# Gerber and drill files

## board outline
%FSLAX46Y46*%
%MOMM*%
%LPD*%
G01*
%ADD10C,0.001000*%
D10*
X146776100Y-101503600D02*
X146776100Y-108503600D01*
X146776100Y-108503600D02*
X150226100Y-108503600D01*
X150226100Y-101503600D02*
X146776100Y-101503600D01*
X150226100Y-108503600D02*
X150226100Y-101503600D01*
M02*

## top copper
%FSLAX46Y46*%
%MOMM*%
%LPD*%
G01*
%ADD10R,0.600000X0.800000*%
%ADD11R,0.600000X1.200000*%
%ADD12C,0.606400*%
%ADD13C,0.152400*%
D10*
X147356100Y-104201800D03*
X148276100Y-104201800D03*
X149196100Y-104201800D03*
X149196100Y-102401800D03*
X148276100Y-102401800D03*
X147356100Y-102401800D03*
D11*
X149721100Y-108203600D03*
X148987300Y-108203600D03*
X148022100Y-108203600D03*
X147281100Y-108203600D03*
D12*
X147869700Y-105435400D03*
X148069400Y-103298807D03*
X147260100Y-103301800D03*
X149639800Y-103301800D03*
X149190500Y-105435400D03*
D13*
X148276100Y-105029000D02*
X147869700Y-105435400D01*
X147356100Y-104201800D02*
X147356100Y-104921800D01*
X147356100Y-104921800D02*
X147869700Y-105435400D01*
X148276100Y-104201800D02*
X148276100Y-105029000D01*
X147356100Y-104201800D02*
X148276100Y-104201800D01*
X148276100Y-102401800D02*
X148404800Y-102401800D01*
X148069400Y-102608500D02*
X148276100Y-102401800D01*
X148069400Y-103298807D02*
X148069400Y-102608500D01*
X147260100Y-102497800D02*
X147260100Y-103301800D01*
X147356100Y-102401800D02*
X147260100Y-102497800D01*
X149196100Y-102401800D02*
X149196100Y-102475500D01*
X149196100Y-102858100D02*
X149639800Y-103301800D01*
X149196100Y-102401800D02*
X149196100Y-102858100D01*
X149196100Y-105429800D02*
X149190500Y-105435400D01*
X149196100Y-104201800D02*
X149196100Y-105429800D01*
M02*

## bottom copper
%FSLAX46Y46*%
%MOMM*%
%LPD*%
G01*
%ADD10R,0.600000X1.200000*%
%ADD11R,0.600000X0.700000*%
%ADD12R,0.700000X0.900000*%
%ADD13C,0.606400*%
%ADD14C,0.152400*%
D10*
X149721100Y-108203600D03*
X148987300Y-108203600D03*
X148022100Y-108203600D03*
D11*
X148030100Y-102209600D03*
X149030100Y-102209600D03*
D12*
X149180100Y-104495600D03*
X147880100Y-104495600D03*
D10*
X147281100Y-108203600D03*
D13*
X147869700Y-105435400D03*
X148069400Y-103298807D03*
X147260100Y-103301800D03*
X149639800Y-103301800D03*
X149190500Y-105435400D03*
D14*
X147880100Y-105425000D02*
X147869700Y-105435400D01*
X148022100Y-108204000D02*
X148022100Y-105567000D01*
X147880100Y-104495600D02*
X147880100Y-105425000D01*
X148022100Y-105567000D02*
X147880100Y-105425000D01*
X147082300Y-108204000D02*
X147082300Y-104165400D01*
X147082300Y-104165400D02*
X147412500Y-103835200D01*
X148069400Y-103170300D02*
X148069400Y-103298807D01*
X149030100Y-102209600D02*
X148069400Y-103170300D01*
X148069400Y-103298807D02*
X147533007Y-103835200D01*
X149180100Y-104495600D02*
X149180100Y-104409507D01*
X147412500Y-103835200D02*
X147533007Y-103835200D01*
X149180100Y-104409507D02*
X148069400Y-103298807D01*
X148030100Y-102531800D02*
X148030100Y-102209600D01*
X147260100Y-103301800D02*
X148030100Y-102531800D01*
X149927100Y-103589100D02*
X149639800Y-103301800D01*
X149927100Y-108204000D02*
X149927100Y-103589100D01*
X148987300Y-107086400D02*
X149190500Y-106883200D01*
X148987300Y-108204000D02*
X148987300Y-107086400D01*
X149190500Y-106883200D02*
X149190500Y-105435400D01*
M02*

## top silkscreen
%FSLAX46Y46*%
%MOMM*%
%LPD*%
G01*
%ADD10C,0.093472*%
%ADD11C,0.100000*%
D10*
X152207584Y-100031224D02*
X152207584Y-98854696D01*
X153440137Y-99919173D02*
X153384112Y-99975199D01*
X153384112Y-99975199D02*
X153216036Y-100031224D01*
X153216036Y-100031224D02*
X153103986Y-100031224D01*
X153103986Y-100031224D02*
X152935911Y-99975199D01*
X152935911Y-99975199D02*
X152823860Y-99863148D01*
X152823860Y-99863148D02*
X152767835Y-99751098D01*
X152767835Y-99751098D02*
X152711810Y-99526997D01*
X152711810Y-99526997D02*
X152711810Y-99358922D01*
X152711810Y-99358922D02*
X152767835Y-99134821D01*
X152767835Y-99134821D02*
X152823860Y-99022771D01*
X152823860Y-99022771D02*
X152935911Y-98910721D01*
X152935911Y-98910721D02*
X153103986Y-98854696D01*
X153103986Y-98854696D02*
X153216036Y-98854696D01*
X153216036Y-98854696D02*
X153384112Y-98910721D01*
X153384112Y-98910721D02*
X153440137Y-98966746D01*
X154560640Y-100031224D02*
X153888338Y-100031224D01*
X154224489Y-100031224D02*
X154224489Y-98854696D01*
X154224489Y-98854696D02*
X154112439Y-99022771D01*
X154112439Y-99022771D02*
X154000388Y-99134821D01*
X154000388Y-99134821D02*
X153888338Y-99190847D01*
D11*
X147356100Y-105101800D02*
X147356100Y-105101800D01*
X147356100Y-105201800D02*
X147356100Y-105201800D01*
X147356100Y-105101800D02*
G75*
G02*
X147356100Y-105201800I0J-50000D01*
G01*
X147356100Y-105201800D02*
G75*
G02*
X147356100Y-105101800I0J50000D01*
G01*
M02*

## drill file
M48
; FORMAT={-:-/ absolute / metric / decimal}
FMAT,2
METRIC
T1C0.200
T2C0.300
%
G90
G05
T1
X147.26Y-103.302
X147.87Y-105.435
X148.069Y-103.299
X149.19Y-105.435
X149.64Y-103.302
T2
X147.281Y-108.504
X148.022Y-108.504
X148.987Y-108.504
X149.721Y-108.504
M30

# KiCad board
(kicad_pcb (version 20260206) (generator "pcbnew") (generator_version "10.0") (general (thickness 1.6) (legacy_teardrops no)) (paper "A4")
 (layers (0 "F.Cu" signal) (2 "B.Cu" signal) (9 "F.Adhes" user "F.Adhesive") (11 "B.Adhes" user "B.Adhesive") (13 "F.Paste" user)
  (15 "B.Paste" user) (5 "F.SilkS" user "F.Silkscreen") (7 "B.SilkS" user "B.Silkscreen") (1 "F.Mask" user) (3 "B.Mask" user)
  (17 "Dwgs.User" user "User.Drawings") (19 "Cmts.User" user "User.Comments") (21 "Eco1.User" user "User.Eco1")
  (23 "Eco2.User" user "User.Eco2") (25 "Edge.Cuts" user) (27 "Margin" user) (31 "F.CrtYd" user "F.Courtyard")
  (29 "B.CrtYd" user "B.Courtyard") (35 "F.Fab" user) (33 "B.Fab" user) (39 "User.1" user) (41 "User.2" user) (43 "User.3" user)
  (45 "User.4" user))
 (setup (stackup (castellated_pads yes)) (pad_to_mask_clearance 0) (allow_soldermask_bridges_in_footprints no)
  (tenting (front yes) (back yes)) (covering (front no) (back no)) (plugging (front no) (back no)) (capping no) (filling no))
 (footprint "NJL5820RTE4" (layer "F.Cu") (at 148.2761 103.3018)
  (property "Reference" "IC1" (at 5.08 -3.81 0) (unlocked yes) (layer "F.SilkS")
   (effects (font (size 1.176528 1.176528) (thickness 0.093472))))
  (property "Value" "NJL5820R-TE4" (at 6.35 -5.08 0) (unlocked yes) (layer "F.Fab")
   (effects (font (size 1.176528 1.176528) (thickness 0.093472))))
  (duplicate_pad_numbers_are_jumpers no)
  (fp_line (start -0.92 1.8) (end -0.92 1.8) (stroke (width 0.1) (type solid)) (layer "F.SilkS"))
  (fp_line (start -0.92 1.9) (end -0.92 1.9) (stroke (width 0.1) (type solid)) (layer "F.SilkS"))
  (fp_arc (start -0.92 1.8) (mid -0.87 1.85) (end -0.92 1.9) (stroke (width 0.1) (type solid)) (layer "F.SilkS"))
  (fp_arc (start -0.92 1.9) (mid -0.97 1.85) (end -0.92 1.8) (stroke (width 0.1) (type solid)) (layer "F.SilkS"))
  (pad "1" smd rect (at -0.92 0.9 90) (size 0.8 0.6) (layers "F.Cu" "F.Mask" "F.Paste") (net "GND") (solder_mask_margin 0.1016)
   (solder_paste_margin 0) (thermal_bridge_angle 0))
  (pad "2" smd rect (at 0 0.9 90) (size 0.8 0.6) (layers "F.Cu" "F.Mask" "F.Paste") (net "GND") (solder_mask_margin 0.1016)
   (solder_paste_margin 0) (thermal_bridge_angle 0))
  (pad "3" smd rect (at 0.92 0.9 90) (size 0.8 0.6) (layers "F.Cu" "F.Mask" "F.Paste") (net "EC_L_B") (solder_mask_margin 0.1016)
   (solder_paste_margin 0) (thermal_bridge_angle 0))
  (pad "4" smd rect (at 0.92 -0.9 90) (size 0.8 0.6) (layers "F.Cu" "F.Mask" "F.Paste") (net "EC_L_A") (solder_mask_margin 0.1016)
   (solder_paste_margin 0) (thermal_bridge_angle 0))
  (pad "5" smd rect (at 0 -0.9 90) (size 0.8 0.6) (layers "F.Cu" "F.Mask" "F.Paste") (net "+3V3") (solder_mask_margin 0.1016)
   (solder_paste_margin 0) (thermal_bridge_angle 0))
  (pad "6" smd rect (at -0.92 -0.9 90) (size 0.8 0.6) (layers "F.Cu" "F.Mask" "F.Paste") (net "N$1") (solder_mask_margin 0.1016)
   (solder_paste_margin 0) (thermal_bridge_angle 0)))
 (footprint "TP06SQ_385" (layer "B.Cu") (at 149.9271 108.204 180)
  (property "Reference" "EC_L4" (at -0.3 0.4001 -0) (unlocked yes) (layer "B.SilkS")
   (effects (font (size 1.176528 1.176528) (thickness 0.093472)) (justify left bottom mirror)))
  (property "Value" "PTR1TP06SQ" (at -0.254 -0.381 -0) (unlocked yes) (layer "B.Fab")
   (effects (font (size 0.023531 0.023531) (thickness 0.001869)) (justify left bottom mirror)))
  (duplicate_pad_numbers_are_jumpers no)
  (pad "TP" thru_hole rect (at 0.2060 -0.2996 180) (size 0.6 1.2) (drill 0.3 (offset 0 0.3000)) (layers "*.Cu" "*.Mask") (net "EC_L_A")
   (solder_mask_margin 0) (solder_paste_margin 0) (thermal_bridge_angle 0)))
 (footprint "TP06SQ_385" (layer "B.Cu") (at 148.9873 108.204 180)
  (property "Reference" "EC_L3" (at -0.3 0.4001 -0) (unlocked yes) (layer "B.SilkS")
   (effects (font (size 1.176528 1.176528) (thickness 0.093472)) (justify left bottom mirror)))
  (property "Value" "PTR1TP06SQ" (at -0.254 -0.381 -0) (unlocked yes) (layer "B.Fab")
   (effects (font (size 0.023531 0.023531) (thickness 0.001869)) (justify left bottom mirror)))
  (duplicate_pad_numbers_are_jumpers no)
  (pad "TP" thru_hole rect (at 0 -0.2996 180) (size 0.6 1.2) (drill 0.3 (offset 0 0.3000)) (layers "*.Cu" "*.Mask") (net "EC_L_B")
   (solder_mask_margin 0) (solder_paste_margin 0) (thermal_bridge_angle 0)))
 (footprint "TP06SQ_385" (layer "B.Cu") (at 148.0221 108.204 180)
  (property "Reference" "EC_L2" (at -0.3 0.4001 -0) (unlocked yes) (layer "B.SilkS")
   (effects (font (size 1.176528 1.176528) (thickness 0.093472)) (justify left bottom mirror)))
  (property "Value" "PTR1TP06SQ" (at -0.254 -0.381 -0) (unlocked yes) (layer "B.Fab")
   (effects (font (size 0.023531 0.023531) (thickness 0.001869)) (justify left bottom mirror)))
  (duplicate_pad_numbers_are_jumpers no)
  (pad "TP" thru_hole rect (at 0 -0.2996 180) (size 0.6 1.2) (drill 0.3 (offset 0 0.3000)) (layers "*.Cu" "*.Mask") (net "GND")
   (solder_mask_margin 0) (solder_paste_margin 0) (thermal_bridge_angle 0)))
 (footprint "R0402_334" (layer "B.Cu") (at 148.5301 102.2096)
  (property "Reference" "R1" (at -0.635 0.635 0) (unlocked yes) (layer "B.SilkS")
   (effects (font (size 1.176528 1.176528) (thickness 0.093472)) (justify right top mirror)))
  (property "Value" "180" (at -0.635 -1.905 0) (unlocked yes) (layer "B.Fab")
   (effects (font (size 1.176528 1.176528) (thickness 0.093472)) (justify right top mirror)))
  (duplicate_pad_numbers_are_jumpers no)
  (pad "1" smd rect (at -0.5 0) (size 0.6 0.7) (layers "B.Cu" "B.Mask" "B.Paste") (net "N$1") (solder_mask_margin 0.1016)
   (solder_paste_margin 0) (thermal_bridge_angle 0))
  (pad "2" smd rect (at 0.5 0) (size 0.6 0.7) (layers "B.Cu" "B.Mask" "B.Paste") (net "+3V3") (solder_mask_margin 0.1016)
   (solder_paste_margin 0) (thermal_bridge_angle 0)))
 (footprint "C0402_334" (layer "B.Cu") (at 148.5301 104.4956 180)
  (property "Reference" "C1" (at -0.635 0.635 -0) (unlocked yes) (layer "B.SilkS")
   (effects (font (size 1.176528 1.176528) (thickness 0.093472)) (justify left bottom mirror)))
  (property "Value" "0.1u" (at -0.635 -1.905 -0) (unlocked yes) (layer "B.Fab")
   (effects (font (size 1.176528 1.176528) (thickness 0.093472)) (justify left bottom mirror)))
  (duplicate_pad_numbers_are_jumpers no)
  (pad "1" smd rect (at -0.65 0 180) (size 0.7 0.9) (layers "B.Cu" "B.Mask" "B.Paste") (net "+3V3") (solder_mask_margin 0.1016)
   (solder_paste_margin 0) (thermal_bridge_angle 0))
  (pad "2" smd rect (at 0.65 0 180) (size 0.7 0.9) (layers "B.Cu" "B.Mask" "B.Paste") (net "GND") (solder_mask_margin 0.1016)
   (solder_paste_margin 0) (thermal_bridge_angle 0)))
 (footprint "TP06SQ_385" (layer "B.Cu") (at 147.0823 108.204 180)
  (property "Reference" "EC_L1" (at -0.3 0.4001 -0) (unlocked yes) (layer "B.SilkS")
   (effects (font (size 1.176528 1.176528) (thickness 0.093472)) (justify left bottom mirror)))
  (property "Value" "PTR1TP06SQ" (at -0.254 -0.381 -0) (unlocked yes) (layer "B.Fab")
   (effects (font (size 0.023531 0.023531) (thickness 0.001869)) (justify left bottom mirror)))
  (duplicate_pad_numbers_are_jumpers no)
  (pad "TP" thru_hole rect (at -0.1988 -0.2996 180) (size 0.6 1.2) (drill 0.3 (offset 0 0.3000)) (layers "*.Cu" "*.Mask") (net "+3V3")
   (solder_mask_margin 0) (solder_paste_margin 0) (thermal_bridge_angle 0)))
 (gr_line (start 146.7761 101.5036) (end 146.7761 108.5036) (stroke (width 0.001) (type solid)) (layer "Edge.Cuts"))
 (gr_line (start 146.7761 108.5036) (end 150.2261 108.5036) (stroke (width 0.001) (type solid)) (layer "Edge.Cuts"))
 (gr_line (start 150.2261 101.5036) (end 146.7761 101.5036) (stroke (width 0.001) (type solid)) (layer "Edge.Cuts"))
 (gr_line (start 150.2261 108.5036) (end 150.2261 101.5036) (stroke (width 0.001) (type solid)) (layer "Edge.Cuts"))
 (segment (start 148.2761 105.029) (end 147.8697 105.4354) (width 0.1524) (layer "F.Cu") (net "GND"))
 (segment (start 147.3561 104.2018) (end 147.3561 104.9218) (width 0.1524) (layer "F.Cu") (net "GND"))
 (segment (start 147.3561 104.9218) (end 147.8697 105.4354) (width 0.1524) (layer "F.Cu") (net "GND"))
 (segment (start 148.2761 104.2018) (end 148.2761 105.029) (width 0.1524) (layer "F.Cu") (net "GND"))
 (segment (start 147.3561 104.2018) (end 148.2761 104.2018) (width 0.1524) (layer "F.Cu") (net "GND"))
 (via (at 147.8697 105.4354) (size 0.6064) (drill 0.2) (layers "F.Cu" "B.Cu") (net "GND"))
 (segment (start 147.8801 105.425) (end 147.8697 105.4354) (width 0.1524) (layer "B.Cu") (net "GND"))
 (segment (start 148.0221 108.204) (end 148.0221 105.567) (width 0.1524) (layer "B.Cu") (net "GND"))
 (segment (start 147.8801 104.4956) (end 147.8801 105.425) (width 0.1524) (layer "B.Cu") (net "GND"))
 (segment (start 148.0221 105.567) (end 147.8801 105.425) (width 0.1524) (layer "B.Cu") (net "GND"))
 (segment (start 148.2761 102.4018) (end 148.4048 102.4018) (width 0.1524) (layer "F.Cu") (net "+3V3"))
 (segment (start 148.0694 102.6085) (end 148.2761 102.4018) (width 0.1524) (layer "F.Cu") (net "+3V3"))
 (segment (start 148.0694 103.298807) (end 148.0694 102.6085) (width 0.1524) (layer "F.Cu") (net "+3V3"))
 (via (at 148.0694 103.298807) (size 0.6064) (drill 0.2) (layers "F.Cu" "B.Cu") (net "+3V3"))
 (segment (start 147.0823 108.204) (end 147.0823 104.1654) (width 0.1524) (layer "B.Cu") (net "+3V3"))
 (segment (start 147.0823 104.1654) (end 147.4125 103.8352) (width 0.1524) (layer "B.Cu") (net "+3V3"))
 (segment (start 148.0694 103.1703) (end 148.0694 103.298807) (width 0.1524) (layer "B.Cu") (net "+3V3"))
 (segment (start 149.0301 102.2096) (end 148.0694 103.1703) (width 0.1524) (layer "B.Cu") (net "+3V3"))
 (segment (start 148.0694 103.298807) (end 147.533007 103.8352) (width 0.1524) (layer "B.Cu") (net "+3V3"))
 (segment (start 149.1801 104.4956) (end 149.1801 104.409507) (width 0.1524) (layer "B.Cu") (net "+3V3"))
 (segment (start 147.4125 103.8352) (end 147.533007 103.8352) (width 0.1524) (layer "B.Cu") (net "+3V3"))
 (segment (start 149.1801 104.409507) (end 148.0694 103.298807) (width 0.1524) (layer "B.Cu") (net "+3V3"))
 (segment (start 147.2601 102.4978) (end 147.2601 103.3018) (width 0.1524) (layer "F.Cu") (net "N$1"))
 (segment (start 147.3561 102.4018) (end 147.2601 102.4978) (width 0.1524) (layer "F.Cu") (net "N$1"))
 (via (at 147.2601 103.3018) (size 0.6064) (drill 0.2) (layers "F.Cu" "B.Cu") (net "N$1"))
 (segment (start 148.0301 102.5318) (end 148.0301 102.2096) (width 0.1524) (layer "B.Cu") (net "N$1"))
 (segment (start 147.2601 103.3018) (end 148.0301 102.5318) (width 0.1524) (layer "B.Cu") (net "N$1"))
 (segment (start 149.1961 102.4018) (end 149.1961 102.4755) (width 0.1524) (layer "F.Cu") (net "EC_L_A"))
 (segment (start 149.1961 102.8581) (end 149.6398 103.3018) (width 0.1524) (layer "F.Cu") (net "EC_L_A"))
 (segment (start 149.1961 102.4018) (end 149.1961 102.8581) (width 0.1524) (layer "F.Cu") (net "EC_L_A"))
 (via (at 149.6398 103.3018) (size 0.6064) (drill 0.2) (layers "F.Cu" "B.Cu") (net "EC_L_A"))
 (segment (start 149.9271 103.5891) (end 149.6398 103.3018) (width 0.1524) (layer "B.Cu") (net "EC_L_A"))
 (segment (start 149.9271 108.204) (end 149.9271 103.5891) (width 0.1524) (layer "B.Cu") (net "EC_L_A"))
 (segment (start 149.1961 105.4298) (end 149.1905 105.4354) (width 0.1524) (layer "F.Cu") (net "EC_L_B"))
 (segment (start 149.1961 104.2018) (end 149.1961 105.4298) (width 0.1524) (layer "F.Cu") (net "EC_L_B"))
 (via (at 149.1905 105.4354) (size 0.6064) (drill 0.2) (layers "F.Cu" "B.Cu") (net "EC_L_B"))
 (segment (start 148.9873 107.0864) (end 149.1905 106.8832) (width 0.1524) (layer "B.Cu") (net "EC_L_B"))
 (segment (start 148.9873 108.204) (end 148.9873 107.0864) (width 0.1524) (layer "B.Cu") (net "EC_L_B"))
 (segment (start 149.1905 106.8832) (end 149.1905 105.4354) (width 0.1524) (layer "B.Cu") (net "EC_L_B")))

